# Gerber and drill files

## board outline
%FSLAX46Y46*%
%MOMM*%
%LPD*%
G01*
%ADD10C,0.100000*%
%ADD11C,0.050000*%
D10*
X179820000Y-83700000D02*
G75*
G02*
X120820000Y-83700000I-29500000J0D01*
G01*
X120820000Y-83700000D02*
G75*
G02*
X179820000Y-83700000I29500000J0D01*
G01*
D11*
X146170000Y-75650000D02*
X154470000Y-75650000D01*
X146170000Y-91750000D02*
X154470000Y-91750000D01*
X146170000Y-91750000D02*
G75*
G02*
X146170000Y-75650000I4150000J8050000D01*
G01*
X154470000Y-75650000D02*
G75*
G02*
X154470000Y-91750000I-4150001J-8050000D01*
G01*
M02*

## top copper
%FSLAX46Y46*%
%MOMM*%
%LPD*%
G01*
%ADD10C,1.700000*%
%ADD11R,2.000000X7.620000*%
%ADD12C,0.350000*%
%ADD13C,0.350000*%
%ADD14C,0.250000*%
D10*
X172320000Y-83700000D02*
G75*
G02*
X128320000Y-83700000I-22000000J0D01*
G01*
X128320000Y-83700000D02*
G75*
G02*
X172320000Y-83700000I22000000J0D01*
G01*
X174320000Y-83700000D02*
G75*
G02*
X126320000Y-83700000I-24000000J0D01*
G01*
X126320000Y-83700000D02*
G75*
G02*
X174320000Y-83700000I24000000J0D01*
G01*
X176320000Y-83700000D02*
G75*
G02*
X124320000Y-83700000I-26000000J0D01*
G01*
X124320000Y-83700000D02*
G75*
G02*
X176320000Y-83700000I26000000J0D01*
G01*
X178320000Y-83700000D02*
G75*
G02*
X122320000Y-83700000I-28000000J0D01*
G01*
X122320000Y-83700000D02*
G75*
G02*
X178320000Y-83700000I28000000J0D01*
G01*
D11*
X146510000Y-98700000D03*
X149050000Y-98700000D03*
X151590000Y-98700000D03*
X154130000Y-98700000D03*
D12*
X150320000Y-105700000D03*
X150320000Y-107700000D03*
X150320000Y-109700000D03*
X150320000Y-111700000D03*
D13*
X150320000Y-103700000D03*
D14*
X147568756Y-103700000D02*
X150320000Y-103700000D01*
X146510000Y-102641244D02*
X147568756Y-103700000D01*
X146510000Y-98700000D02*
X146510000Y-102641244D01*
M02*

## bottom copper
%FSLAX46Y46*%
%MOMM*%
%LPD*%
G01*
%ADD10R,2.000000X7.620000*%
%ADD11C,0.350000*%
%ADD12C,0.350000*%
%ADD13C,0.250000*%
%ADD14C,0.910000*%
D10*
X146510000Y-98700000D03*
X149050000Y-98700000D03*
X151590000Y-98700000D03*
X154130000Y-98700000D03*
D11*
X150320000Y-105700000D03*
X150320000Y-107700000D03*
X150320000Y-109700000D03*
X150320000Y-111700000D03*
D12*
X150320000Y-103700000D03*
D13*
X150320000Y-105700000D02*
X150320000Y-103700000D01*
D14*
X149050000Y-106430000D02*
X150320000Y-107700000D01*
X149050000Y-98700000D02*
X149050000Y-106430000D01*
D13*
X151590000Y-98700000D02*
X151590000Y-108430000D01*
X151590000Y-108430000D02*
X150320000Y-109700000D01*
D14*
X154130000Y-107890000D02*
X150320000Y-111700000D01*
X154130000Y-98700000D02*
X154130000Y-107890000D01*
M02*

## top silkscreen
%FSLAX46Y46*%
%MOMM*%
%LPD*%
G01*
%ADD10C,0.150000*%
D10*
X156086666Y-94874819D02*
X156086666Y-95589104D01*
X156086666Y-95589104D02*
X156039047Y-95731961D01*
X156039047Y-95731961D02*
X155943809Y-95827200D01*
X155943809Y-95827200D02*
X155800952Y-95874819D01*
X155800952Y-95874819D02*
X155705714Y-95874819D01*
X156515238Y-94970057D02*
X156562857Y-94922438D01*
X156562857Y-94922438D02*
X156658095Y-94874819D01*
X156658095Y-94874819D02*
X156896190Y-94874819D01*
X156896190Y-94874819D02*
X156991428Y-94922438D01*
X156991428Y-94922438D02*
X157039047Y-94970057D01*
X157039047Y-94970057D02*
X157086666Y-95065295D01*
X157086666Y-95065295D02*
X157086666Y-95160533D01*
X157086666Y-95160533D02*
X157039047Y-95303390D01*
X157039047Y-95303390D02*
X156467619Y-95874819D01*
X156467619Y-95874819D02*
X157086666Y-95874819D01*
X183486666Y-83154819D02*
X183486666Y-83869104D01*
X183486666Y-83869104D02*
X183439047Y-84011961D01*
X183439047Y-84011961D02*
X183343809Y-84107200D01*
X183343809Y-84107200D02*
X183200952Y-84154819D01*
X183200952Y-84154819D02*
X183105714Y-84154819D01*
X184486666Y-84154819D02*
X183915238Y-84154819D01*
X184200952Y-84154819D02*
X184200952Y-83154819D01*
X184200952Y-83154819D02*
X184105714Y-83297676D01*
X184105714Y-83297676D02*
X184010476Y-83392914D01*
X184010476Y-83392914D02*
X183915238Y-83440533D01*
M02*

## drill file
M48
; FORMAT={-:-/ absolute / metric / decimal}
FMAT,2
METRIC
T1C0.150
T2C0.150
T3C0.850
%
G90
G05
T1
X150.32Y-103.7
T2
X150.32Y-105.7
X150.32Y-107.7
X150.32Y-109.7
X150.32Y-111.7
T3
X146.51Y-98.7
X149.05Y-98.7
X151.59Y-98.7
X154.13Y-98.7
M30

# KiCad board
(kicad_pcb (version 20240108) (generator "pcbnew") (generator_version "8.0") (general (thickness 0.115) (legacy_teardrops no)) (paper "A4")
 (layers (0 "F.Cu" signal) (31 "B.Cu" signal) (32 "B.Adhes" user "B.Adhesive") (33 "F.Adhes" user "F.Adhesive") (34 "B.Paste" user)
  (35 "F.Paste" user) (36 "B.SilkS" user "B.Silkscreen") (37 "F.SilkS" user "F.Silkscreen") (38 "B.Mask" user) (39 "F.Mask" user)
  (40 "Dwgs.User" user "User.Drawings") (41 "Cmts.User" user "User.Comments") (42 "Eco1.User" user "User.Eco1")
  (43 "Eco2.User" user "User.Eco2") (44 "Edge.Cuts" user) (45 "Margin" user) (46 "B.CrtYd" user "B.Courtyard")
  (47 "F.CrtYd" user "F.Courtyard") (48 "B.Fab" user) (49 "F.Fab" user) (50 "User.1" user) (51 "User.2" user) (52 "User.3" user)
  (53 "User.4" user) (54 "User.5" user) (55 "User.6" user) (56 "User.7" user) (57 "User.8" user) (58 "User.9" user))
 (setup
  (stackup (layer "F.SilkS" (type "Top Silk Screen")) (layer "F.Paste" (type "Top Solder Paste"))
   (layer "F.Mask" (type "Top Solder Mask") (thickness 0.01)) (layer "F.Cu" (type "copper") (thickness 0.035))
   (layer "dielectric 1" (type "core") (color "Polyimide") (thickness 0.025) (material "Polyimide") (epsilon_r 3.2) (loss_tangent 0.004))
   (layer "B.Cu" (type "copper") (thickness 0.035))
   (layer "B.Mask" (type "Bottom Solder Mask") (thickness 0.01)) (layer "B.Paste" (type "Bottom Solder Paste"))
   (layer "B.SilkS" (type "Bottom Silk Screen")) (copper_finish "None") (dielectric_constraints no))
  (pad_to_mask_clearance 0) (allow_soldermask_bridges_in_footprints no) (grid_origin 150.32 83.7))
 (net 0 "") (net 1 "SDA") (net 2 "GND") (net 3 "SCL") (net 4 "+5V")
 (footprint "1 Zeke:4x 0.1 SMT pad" (layer "F.Cu") (at 154.13 98.7 90)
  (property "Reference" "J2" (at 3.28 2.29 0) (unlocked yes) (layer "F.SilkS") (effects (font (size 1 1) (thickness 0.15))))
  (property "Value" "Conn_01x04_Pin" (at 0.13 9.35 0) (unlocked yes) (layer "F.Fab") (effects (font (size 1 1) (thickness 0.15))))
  (pad "1" thru_hole rect (at 0 -7.62 90) (size 7.62 2) (drill 0.85) (layers "*.Cu" "*.Mask") (remove_unused_layers no) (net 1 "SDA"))
  (pad "2" thru_hole rect (at 0 -5.08 90) (size 7.62 2) (drill 0.85) (layers "*.Cu" "*.Mask") (remove_unused_layers no) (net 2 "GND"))
  (pad "3" thru_hole rect (at 0 -2.54 90) (size 7.62 2) (drill 0.85) (layers "*.Cu" "*.Mask") (remove_unused_layers no) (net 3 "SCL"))
  (pad "4" thru_hole rect (at 0 0 90) (size 7.62 2) (drill 0.85) (layers "*.Cu" "*.Mask") (remove_unused_layers no) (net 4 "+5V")))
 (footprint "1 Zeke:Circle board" (layer "F.Cu") (at 150.32 83.7)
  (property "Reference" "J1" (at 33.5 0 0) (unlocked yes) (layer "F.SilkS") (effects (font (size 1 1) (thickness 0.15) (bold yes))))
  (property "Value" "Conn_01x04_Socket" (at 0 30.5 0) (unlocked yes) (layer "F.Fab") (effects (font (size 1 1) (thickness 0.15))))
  (fp_circle (center 0 0) (end 22 0) (stroke (width 1.7) (type solid)) (fill none) (layer "F.Cu"))
  (fp_circle (center 0 0) (end 24 0) (stroke (width 1.7) (type solid)) (fill none) (layer "F.Cu"))
  (fp_circle (center 0 0) (end 26 0) (stroke (width 1.7) (type solid)) (fill none) (layer "F.Cu"))
  (fp_circle (center 0 0) (end 28 0) (stroke (width 1.7) (type solid)) (fill none) (layer "F.Cu"))
  (fp_line (start -4.15 -8.05) (end 4.15 -8.05) (stroke (width 0.05) (type default)) (layer "Edge.Cuts"))
  (fp_line (start -4.15 8.05) (end 4.15 8.05) (stroke (width 0.05) (type default)) (layer "Edge.Cuts"))
  (fp_arc (start -4.15 8.05) (mid -9.056765 0) (end -4.15 -8.05) (stroke (width 0.05) (type default)) (layer "Edge.Cuts"))
  (fp_arc (start 4.15 -8.05) (mid 9.056765 0) (end 4.15 8.05) (stroke (width 0.05) (type default)) (layer "Edge.Cuts"))
  (pad "1" thru_hole circle (at 0 22) (size 0.35 0.35) (drill 0.15) (layers "*.Cu" "*.Mask") (remove_unused_layers no) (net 1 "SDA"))
  (pad "2" thru_hole circle (at 0 24) (size 0.35 0.35) (drill 0.15) (layers "*.Cu" "*.Mask") (remove_unused_layers no) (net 2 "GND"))
  (pad "3" thru_hole circle (at 0 26) (size 0.35 0.35) (drill 0.15) (layers "*.Cu" "*.Mask") (remove_unused_layers no) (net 3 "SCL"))
  (pad "4" thru_hole circle (at 0 28) (size 0.35 0.35) (drill 0.15) (layers "*.Cu" "*.Mask") (remove_unused_layers no) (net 4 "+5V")))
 (gr_circle (center 150.32 83.7) (end 179.82 83.7) (stroke (width 0.1) (type default)) (fill none) (layer "Edge.Cuts"))
 (segment (start 147.568756 103.7) (end 150.32 103.7) (width 0.25) (layer "F.Cu") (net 1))
 (segment (start 146.51 102.641244) (end 147.568756 103.7) (width 0.25) (layer "F.Cu") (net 1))
 (segment (start 146.51 98.7) (end 146.51 102.641244) (width 0.25) (layer "F.Cu") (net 1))
 (via (at 150.32 103.7) (size 0.35) (drill 0.15) (layers "F.Cu" "B.Cu") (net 1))
 (segment (start 150.32 105.7) (end 150.32 103.7) (width 0.25) (layer "B.Cu") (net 1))
 (segment (start 149.05 106.43) (end 150.32 107.7) (width 0.91) (layer "B.Cu") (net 2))
 (segment (start 149.05 98.7) (end 149.05 106.43) (width 0.91) (layer "B.Cu") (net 2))
 (segment (start 151.59 98.7) (end 151.59 108.43) (width 0.25) (layer "B.Cu") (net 3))
 (segment (start 151.59 108.43) (end 150.32 109.7) (width 0.25) (layer "B.Cu") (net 3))
 (segment (start 154.13 107.89) (end 150.32 111.7) (width 0.91) (layer "B.Cu") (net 4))
 (segment (start 154.13 98.7) (end 154.13 107.89) (width 0.91) (layer "B.Cu") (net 4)))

